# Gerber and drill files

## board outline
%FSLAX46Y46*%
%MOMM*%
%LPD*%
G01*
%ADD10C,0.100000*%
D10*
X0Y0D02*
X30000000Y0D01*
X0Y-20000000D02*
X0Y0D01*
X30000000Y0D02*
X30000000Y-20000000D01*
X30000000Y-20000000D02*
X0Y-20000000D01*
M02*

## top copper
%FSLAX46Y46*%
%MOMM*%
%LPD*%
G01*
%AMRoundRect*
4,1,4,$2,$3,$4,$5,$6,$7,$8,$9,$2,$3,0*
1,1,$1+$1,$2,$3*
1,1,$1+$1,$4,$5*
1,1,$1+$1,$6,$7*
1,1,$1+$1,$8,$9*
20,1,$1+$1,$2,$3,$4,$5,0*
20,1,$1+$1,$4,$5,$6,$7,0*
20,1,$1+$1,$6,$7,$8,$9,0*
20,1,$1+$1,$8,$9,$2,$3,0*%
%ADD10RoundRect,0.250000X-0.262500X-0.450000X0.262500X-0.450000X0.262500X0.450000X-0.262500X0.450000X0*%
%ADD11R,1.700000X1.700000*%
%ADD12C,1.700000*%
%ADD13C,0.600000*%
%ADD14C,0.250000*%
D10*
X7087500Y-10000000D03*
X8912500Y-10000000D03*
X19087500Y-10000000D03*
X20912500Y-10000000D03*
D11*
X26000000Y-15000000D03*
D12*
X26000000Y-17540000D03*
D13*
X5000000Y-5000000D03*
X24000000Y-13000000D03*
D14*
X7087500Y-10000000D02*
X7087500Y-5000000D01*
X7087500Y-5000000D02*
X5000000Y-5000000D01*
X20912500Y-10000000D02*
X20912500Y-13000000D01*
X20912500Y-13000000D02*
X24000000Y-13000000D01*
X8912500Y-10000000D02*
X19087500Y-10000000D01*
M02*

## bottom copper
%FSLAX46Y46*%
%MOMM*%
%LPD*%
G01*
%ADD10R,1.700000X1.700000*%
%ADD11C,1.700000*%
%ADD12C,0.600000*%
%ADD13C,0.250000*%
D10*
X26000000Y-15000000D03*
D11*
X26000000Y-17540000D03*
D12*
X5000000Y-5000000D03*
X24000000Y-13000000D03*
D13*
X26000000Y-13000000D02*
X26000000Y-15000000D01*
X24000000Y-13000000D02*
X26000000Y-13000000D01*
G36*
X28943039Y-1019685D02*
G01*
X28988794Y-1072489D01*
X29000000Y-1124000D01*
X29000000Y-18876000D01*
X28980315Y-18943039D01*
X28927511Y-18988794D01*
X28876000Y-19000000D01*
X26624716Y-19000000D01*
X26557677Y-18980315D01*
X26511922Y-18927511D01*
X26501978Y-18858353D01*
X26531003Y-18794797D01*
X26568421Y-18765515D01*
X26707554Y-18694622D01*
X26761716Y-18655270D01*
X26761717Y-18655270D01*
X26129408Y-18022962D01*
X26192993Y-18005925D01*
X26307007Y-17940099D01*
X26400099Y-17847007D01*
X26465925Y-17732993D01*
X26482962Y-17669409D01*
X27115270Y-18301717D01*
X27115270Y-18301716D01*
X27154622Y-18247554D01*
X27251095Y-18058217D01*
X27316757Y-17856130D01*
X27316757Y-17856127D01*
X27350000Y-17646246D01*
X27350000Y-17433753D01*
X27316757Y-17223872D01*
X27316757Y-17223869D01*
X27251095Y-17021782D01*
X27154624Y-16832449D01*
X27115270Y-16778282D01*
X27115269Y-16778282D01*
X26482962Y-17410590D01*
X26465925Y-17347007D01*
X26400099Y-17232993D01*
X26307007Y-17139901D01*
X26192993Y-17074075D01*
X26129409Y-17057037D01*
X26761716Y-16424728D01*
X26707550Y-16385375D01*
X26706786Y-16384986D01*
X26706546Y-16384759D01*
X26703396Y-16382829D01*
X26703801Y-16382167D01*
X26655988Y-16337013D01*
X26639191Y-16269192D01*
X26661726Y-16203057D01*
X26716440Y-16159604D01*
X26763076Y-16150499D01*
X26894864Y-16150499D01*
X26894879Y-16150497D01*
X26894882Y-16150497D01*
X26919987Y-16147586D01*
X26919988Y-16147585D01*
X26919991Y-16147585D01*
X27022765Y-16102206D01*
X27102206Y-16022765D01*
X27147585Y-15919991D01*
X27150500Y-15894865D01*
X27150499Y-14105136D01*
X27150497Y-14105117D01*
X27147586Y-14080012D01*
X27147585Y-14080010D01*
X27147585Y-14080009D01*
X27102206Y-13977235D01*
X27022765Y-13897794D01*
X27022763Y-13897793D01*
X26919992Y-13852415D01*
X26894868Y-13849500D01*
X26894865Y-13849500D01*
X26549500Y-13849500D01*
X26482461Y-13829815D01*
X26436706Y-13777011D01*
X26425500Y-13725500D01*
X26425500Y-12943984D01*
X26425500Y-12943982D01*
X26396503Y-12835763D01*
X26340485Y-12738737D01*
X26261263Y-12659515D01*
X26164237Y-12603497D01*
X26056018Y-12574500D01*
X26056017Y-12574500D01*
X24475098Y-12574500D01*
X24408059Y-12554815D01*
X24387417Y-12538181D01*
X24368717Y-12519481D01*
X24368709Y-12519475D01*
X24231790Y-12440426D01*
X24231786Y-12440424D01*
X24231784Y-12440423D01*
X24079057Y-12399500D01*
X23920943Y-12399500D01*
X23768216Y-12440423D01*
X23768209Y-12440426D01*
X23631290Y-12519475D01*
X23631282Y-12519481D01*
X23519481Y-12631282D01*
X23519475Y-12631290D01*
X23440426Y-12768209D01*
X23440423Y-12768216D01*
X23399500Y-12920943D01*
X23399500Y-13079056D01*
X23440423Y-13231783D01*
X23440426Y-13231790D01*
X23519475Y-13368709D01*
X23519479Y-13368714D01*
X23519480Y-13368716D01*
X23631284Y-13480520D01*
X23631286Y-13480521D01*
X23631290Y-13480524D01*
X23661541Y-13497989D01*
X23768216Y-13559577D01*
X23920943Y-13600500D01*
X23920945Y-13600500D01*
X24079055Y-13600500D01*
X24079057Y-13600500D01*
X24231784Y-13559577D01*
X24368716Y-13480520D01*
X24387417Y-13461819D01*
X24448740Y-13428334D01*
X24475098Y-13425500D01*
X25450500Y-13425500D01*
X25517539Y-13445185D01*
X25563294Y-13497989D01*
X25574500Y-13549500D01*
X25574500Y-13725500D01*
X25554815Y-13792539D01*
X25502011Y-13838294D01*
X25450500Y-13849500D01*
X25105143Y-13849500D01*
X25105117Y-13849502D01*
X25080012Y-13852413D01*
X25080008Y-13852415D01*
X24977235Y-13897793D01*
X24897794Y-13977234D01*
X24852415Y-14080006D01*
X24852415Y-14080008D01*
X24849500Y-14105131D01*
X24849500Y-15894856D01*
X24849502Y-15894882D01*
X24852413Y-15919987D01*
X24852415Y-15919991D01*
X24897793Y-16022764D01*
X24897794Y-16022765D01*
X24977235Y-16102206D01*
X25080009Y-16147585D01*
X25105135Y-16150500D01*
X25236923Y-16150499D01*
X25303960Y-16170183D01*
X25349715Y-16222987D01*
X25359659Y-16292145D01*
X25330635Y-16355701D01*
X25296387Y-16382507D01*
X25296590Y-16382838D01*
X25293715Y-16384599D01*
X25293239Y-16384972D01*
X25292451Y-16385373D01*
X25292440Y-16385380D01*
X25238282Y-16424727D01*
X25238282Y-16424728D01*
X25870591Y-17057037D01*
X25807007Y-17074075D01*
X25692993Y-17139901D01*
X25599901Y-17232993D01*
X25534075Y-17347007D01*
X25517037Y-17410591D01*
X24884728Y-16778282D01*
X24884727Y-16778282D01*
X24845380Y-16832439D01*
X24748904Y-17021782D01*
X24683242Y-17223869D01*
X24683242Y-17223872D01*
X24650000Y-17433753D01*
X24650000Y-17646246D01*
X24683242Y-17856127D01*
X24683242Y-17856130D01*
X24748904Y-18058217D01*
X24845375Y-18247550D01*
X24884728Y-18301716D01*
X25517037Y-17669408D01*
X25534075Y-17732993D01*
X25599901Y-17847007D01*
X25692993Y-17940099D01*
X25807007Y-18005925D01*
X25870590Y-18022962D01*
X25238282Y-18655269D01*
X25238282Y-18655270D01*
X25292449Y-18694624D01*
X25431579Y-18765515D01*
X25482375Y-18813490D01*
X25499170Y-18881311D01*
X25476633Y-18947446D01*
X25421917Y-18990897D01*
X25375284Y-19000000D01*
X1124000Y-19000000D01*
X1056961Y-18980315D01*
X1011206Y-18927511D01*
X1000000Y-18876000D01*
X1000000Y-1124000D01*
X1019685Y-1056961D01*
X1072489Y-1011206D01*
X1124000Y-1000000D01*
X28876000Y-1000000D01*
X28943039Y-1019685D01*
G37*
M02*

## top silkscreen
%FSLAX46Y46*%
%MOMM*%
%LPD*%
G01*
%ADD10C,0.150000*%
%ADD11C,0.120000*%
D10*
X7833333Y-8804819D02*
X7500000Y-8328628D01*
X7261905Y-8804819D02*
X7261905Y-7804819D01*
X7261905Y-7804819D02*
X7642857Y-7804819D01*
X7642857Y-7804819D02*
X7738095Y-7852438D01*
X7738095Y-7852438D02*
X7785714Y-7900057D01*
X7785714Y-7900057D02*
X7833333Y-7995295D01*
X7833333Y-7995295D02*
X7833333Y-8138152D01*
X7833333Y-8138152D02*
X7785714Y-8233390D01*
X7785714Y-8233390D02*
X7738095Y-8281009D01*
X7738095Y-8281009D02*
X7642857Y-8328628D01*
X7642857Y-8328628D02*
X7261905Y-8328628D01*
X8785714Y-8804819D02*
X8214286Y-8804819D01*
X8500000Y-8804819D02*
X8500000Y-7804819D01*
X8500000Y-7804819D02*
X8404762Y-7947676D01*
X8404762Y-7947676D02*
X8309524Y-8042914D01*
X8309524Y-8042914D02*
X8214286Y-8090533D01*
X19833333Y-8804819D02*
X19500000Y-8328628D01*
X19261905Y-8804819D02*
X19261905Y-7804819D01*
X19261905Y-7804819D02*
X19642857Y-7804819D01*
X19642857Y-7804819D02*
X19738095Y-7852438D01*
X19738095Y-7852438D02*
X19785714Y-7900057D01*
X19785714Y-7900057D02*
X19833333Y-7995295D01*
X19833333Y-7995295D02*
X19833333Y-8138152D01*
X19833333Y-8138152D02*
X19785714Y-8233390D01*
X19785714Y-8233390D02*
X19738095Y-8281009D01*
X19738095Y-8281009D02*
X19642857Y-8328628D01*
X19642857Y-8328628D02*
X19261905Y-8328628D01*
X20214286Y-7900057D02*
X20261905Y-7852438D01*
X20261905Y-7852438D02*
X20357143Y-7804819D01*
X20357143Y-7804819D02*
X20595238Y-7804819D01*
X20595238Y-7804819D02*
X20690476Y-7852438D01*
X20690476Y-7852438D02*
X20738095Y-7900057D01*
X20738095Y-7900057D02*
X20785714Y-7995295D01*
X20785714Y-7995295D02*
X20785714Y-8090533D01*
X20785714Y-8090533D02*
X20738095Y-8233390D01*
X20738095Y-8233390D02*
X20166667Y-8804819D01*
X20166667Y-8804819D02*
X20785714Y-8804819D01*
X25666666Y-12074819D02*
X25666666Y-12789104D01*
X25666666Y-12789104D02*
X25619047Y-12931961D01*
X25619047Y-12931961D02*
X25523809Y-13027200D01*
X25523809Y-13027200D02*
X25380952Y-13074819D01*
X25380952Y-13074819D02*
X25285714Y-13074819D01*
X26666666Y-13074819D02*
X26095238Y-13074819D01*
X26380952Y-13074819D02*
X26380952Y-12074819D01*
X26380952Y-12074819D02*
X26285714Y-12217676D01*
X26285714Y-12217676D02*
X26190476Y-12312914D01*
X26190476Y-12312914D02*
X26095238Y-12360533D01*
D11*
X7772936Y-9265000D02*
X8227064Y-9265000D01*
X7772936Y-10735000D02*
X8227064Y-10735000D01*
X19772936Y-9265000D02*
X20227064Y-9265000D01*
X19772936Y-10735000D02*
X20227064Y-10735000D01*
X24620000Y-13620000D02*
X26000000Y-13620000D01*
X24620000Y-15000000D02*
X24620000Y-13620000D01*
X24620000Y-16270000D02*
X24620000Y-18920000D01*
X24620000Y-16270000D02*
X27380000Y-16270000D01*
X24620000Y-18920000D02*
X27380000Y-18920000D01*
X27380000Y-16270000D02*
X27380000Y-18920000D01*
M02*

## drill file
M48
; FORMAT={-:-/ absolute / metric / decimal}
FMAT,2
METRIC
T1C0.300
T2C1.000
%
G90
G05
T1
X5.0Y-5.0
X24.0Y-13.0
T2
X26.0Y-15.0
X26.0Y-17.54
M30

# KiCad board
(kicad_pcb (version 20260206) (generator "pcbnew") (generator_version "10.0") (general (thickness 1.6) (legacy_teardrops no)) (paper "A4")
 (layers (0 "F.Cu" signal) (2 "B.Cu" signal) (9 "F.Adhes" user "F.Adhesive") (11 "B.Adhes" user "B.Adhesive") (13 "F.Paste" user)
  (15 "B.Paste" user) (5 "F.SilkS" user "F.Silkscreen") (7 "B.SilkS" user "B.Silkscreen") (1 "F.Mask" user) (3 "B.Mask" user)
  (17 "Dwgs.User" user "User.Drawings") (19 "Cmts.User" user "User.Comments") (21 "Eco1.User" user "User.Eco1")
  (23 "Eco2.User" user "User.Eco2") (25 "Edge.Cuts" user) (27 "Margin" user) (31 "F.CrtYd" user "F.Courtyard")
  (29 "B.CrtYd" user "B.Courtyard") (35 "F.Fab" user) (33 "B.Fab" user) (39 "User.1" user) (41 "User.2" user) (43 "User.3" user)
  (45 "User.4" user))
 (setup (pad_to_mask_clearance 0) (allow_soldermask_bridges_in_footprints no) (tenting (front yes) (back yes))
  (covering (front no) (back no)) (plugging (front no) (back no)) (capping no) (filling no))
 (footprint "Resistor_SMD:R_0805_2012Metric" (layer "F.Cu") (at 8 10)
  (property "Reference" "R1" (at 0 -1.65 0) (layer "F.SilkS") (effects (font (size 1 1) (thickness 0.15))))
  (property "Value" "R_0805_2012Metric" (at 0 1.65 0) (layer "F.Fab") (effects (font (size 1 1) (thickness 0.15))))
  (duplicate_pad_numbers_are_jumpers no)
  (fp_line (start -0.227064 -0.735) (end 0.227064 -0.735) (stroke (width 0.12) (type solid)) (layer "F.SilkS"))
  (fp_line (start -0.227064 0.735) (end 0.227064 0.735) (stroke (width 0.12) (type solid)) (layer "F.SilkS"))
  (pad "1" smd roundrect (at -0.9125 0) (size 1.025 1.4) (layers "F.Cu" "F.Mask" "F.Paste") (roundrect_rratio 0.243902) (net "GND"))
  (pad "2" smd roundrect (at 0.9125 0) (size 1.025 1.4) (layers "F.Cu" "F.Mask" "F.Paste") (roundrect_rratio 0.243902) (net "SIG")))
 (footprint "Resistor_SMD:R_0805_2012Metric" (layer "F.Cu") (at 20 10)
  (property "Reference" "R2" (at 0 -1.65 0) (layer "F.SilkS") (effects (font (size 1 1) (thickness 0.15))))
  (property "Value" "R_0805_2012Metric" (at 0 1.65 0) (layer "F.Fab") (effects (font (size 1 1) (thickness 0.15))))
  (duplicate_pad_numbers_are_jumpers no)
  (fp_line (start -0.227064 -0.735) (end 0.227064 -0.735) (stroke (width 0.12) (type solid)) (layer "F.SilkS"))
  (fp_line (start -0.227064 0.735) (end 0.227064 0.735) (stroke (width 0.12) (type solid)) (layer "F.SilkS"))
  (pad "1" smd roundrect (at -0.9125 0) (size 1.025 1.4) (layers "F.Cu" "F.Mask" "F.Paste") (roundrect_rratio 0.243902) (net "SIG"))
  (pad "2" smd roundrect (at 0.9125 0) (size 1.025 1.4) (layers "F.Cu" "F.Mask" "F.Paste") (roundrect_rratio 0.243902) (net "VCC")))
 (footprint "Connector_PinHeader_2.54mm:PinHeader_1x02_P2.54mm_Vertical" (layer "F.Cu") (at 26 15)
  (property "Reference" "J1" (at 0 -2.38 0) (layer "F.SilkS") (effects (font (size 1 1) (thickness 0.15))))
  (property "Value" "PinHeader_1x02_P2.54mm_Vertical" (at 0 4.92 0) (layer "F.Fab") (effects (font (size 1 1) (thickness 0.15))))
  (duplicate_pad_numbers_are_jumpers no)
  (fp_line (start -1.38 -1.38) (end 0 -1.38) (stroke (width 0.12) (type solid)) (layer "F.SilkS"))
  (fp_line (start -1.38 0) (end -1.38 -1.38) (stroke (width 0.12) (type solid)) (layer "F.SilkS"))
  (fp_line (start -1.38 1.27) (end -1.38 3.92) (stroke (width 0.12) (type solid)) (layer "F.SilkS"))
  (fp_line (start -1.38 1.27) (end 1.38 1.27) (stroke (width 0.12) (type solid)) (layer "F.SilkS"))
  (fp_line (start -1.38 3.92) (end 1.38 3.92) (stroke (width 0.12) (type solid)) (layer "F.SilkS"))
  (fp_line (start 1.38 1.27) (end 1.38 3.92) (stroke (width 0.12) (type solid)) (layer "F.SilkS"))
  (pad "1" thru_hole rect (at 0 0) (size 1.7 1.7) (drill 1) (layers "*.Cu" "*.Mask") (remove_unused_layers no) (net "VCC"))
  (pad "2" thru_hole circle (at 0 2.54) (size 1.7 1.7) (drill 1) (layers "*.Cu" "*.Mask") (remove_unused_layers no) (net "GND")))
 (gr_line (start 0 0) (end 30 0) (stroke (width 0.1) (type default)) (layer "Edge.Cuts"))
 (gr_line (start 0 20) (end 0 0) (stroke (width 0.1) (type default)) (layer "Edge.Cuts"))
 (gr_line (start 30 0) (end 30 20) (stroke (width 0.1) (type default)) (layer "Edge.Cuts"))
 (gr_line (start 30 20) (end 0 20) (stroke (width 0.1) (type default)) (layer "Edge.Cuts"))
 (segment (start 7.0875 10) (end 7.0875 5) (width 0.25) (layer "F.Cu") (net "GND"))
 (segment (start 7.0875 5) (end 5 5) (width 0.25) (layer "F.Cu") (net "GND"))
 (via (at 5 5) (size 0.6) (drill 0.3) (layers "F.Cu" "B.Cu") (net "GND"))
 (segment (start 20.9125 10) (end 20.9125 13) (width 0.25) (layer "F.Cu") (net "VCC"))
 (segment (start 20.9125 13) (end 24 13) (width 0.25) (layer "F.Cu") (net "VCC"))
 (via (at 24 13) (size 0.6) (drill 0.3) (layers "F.Cu" "B.Cu") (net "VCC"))
 (segment (start 26 13) (end 26 15) (width 0.25) (layer "B.Cu") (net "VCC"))
 (segment (start 24 13) (end 26 13) (width 0.25) (layer "B.Cu") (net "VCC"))
 (segment (start 8.9125 10) (end 19.0875 10) (width 0.25) (layer "F.Cu") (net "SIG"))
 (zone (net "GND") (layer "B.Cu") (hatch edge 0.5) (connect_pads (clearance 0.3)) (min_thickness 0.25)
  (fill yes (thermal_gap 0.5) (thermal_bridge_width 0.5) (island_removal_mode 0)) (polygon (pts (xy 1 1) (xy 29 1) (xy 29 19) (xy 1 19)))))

